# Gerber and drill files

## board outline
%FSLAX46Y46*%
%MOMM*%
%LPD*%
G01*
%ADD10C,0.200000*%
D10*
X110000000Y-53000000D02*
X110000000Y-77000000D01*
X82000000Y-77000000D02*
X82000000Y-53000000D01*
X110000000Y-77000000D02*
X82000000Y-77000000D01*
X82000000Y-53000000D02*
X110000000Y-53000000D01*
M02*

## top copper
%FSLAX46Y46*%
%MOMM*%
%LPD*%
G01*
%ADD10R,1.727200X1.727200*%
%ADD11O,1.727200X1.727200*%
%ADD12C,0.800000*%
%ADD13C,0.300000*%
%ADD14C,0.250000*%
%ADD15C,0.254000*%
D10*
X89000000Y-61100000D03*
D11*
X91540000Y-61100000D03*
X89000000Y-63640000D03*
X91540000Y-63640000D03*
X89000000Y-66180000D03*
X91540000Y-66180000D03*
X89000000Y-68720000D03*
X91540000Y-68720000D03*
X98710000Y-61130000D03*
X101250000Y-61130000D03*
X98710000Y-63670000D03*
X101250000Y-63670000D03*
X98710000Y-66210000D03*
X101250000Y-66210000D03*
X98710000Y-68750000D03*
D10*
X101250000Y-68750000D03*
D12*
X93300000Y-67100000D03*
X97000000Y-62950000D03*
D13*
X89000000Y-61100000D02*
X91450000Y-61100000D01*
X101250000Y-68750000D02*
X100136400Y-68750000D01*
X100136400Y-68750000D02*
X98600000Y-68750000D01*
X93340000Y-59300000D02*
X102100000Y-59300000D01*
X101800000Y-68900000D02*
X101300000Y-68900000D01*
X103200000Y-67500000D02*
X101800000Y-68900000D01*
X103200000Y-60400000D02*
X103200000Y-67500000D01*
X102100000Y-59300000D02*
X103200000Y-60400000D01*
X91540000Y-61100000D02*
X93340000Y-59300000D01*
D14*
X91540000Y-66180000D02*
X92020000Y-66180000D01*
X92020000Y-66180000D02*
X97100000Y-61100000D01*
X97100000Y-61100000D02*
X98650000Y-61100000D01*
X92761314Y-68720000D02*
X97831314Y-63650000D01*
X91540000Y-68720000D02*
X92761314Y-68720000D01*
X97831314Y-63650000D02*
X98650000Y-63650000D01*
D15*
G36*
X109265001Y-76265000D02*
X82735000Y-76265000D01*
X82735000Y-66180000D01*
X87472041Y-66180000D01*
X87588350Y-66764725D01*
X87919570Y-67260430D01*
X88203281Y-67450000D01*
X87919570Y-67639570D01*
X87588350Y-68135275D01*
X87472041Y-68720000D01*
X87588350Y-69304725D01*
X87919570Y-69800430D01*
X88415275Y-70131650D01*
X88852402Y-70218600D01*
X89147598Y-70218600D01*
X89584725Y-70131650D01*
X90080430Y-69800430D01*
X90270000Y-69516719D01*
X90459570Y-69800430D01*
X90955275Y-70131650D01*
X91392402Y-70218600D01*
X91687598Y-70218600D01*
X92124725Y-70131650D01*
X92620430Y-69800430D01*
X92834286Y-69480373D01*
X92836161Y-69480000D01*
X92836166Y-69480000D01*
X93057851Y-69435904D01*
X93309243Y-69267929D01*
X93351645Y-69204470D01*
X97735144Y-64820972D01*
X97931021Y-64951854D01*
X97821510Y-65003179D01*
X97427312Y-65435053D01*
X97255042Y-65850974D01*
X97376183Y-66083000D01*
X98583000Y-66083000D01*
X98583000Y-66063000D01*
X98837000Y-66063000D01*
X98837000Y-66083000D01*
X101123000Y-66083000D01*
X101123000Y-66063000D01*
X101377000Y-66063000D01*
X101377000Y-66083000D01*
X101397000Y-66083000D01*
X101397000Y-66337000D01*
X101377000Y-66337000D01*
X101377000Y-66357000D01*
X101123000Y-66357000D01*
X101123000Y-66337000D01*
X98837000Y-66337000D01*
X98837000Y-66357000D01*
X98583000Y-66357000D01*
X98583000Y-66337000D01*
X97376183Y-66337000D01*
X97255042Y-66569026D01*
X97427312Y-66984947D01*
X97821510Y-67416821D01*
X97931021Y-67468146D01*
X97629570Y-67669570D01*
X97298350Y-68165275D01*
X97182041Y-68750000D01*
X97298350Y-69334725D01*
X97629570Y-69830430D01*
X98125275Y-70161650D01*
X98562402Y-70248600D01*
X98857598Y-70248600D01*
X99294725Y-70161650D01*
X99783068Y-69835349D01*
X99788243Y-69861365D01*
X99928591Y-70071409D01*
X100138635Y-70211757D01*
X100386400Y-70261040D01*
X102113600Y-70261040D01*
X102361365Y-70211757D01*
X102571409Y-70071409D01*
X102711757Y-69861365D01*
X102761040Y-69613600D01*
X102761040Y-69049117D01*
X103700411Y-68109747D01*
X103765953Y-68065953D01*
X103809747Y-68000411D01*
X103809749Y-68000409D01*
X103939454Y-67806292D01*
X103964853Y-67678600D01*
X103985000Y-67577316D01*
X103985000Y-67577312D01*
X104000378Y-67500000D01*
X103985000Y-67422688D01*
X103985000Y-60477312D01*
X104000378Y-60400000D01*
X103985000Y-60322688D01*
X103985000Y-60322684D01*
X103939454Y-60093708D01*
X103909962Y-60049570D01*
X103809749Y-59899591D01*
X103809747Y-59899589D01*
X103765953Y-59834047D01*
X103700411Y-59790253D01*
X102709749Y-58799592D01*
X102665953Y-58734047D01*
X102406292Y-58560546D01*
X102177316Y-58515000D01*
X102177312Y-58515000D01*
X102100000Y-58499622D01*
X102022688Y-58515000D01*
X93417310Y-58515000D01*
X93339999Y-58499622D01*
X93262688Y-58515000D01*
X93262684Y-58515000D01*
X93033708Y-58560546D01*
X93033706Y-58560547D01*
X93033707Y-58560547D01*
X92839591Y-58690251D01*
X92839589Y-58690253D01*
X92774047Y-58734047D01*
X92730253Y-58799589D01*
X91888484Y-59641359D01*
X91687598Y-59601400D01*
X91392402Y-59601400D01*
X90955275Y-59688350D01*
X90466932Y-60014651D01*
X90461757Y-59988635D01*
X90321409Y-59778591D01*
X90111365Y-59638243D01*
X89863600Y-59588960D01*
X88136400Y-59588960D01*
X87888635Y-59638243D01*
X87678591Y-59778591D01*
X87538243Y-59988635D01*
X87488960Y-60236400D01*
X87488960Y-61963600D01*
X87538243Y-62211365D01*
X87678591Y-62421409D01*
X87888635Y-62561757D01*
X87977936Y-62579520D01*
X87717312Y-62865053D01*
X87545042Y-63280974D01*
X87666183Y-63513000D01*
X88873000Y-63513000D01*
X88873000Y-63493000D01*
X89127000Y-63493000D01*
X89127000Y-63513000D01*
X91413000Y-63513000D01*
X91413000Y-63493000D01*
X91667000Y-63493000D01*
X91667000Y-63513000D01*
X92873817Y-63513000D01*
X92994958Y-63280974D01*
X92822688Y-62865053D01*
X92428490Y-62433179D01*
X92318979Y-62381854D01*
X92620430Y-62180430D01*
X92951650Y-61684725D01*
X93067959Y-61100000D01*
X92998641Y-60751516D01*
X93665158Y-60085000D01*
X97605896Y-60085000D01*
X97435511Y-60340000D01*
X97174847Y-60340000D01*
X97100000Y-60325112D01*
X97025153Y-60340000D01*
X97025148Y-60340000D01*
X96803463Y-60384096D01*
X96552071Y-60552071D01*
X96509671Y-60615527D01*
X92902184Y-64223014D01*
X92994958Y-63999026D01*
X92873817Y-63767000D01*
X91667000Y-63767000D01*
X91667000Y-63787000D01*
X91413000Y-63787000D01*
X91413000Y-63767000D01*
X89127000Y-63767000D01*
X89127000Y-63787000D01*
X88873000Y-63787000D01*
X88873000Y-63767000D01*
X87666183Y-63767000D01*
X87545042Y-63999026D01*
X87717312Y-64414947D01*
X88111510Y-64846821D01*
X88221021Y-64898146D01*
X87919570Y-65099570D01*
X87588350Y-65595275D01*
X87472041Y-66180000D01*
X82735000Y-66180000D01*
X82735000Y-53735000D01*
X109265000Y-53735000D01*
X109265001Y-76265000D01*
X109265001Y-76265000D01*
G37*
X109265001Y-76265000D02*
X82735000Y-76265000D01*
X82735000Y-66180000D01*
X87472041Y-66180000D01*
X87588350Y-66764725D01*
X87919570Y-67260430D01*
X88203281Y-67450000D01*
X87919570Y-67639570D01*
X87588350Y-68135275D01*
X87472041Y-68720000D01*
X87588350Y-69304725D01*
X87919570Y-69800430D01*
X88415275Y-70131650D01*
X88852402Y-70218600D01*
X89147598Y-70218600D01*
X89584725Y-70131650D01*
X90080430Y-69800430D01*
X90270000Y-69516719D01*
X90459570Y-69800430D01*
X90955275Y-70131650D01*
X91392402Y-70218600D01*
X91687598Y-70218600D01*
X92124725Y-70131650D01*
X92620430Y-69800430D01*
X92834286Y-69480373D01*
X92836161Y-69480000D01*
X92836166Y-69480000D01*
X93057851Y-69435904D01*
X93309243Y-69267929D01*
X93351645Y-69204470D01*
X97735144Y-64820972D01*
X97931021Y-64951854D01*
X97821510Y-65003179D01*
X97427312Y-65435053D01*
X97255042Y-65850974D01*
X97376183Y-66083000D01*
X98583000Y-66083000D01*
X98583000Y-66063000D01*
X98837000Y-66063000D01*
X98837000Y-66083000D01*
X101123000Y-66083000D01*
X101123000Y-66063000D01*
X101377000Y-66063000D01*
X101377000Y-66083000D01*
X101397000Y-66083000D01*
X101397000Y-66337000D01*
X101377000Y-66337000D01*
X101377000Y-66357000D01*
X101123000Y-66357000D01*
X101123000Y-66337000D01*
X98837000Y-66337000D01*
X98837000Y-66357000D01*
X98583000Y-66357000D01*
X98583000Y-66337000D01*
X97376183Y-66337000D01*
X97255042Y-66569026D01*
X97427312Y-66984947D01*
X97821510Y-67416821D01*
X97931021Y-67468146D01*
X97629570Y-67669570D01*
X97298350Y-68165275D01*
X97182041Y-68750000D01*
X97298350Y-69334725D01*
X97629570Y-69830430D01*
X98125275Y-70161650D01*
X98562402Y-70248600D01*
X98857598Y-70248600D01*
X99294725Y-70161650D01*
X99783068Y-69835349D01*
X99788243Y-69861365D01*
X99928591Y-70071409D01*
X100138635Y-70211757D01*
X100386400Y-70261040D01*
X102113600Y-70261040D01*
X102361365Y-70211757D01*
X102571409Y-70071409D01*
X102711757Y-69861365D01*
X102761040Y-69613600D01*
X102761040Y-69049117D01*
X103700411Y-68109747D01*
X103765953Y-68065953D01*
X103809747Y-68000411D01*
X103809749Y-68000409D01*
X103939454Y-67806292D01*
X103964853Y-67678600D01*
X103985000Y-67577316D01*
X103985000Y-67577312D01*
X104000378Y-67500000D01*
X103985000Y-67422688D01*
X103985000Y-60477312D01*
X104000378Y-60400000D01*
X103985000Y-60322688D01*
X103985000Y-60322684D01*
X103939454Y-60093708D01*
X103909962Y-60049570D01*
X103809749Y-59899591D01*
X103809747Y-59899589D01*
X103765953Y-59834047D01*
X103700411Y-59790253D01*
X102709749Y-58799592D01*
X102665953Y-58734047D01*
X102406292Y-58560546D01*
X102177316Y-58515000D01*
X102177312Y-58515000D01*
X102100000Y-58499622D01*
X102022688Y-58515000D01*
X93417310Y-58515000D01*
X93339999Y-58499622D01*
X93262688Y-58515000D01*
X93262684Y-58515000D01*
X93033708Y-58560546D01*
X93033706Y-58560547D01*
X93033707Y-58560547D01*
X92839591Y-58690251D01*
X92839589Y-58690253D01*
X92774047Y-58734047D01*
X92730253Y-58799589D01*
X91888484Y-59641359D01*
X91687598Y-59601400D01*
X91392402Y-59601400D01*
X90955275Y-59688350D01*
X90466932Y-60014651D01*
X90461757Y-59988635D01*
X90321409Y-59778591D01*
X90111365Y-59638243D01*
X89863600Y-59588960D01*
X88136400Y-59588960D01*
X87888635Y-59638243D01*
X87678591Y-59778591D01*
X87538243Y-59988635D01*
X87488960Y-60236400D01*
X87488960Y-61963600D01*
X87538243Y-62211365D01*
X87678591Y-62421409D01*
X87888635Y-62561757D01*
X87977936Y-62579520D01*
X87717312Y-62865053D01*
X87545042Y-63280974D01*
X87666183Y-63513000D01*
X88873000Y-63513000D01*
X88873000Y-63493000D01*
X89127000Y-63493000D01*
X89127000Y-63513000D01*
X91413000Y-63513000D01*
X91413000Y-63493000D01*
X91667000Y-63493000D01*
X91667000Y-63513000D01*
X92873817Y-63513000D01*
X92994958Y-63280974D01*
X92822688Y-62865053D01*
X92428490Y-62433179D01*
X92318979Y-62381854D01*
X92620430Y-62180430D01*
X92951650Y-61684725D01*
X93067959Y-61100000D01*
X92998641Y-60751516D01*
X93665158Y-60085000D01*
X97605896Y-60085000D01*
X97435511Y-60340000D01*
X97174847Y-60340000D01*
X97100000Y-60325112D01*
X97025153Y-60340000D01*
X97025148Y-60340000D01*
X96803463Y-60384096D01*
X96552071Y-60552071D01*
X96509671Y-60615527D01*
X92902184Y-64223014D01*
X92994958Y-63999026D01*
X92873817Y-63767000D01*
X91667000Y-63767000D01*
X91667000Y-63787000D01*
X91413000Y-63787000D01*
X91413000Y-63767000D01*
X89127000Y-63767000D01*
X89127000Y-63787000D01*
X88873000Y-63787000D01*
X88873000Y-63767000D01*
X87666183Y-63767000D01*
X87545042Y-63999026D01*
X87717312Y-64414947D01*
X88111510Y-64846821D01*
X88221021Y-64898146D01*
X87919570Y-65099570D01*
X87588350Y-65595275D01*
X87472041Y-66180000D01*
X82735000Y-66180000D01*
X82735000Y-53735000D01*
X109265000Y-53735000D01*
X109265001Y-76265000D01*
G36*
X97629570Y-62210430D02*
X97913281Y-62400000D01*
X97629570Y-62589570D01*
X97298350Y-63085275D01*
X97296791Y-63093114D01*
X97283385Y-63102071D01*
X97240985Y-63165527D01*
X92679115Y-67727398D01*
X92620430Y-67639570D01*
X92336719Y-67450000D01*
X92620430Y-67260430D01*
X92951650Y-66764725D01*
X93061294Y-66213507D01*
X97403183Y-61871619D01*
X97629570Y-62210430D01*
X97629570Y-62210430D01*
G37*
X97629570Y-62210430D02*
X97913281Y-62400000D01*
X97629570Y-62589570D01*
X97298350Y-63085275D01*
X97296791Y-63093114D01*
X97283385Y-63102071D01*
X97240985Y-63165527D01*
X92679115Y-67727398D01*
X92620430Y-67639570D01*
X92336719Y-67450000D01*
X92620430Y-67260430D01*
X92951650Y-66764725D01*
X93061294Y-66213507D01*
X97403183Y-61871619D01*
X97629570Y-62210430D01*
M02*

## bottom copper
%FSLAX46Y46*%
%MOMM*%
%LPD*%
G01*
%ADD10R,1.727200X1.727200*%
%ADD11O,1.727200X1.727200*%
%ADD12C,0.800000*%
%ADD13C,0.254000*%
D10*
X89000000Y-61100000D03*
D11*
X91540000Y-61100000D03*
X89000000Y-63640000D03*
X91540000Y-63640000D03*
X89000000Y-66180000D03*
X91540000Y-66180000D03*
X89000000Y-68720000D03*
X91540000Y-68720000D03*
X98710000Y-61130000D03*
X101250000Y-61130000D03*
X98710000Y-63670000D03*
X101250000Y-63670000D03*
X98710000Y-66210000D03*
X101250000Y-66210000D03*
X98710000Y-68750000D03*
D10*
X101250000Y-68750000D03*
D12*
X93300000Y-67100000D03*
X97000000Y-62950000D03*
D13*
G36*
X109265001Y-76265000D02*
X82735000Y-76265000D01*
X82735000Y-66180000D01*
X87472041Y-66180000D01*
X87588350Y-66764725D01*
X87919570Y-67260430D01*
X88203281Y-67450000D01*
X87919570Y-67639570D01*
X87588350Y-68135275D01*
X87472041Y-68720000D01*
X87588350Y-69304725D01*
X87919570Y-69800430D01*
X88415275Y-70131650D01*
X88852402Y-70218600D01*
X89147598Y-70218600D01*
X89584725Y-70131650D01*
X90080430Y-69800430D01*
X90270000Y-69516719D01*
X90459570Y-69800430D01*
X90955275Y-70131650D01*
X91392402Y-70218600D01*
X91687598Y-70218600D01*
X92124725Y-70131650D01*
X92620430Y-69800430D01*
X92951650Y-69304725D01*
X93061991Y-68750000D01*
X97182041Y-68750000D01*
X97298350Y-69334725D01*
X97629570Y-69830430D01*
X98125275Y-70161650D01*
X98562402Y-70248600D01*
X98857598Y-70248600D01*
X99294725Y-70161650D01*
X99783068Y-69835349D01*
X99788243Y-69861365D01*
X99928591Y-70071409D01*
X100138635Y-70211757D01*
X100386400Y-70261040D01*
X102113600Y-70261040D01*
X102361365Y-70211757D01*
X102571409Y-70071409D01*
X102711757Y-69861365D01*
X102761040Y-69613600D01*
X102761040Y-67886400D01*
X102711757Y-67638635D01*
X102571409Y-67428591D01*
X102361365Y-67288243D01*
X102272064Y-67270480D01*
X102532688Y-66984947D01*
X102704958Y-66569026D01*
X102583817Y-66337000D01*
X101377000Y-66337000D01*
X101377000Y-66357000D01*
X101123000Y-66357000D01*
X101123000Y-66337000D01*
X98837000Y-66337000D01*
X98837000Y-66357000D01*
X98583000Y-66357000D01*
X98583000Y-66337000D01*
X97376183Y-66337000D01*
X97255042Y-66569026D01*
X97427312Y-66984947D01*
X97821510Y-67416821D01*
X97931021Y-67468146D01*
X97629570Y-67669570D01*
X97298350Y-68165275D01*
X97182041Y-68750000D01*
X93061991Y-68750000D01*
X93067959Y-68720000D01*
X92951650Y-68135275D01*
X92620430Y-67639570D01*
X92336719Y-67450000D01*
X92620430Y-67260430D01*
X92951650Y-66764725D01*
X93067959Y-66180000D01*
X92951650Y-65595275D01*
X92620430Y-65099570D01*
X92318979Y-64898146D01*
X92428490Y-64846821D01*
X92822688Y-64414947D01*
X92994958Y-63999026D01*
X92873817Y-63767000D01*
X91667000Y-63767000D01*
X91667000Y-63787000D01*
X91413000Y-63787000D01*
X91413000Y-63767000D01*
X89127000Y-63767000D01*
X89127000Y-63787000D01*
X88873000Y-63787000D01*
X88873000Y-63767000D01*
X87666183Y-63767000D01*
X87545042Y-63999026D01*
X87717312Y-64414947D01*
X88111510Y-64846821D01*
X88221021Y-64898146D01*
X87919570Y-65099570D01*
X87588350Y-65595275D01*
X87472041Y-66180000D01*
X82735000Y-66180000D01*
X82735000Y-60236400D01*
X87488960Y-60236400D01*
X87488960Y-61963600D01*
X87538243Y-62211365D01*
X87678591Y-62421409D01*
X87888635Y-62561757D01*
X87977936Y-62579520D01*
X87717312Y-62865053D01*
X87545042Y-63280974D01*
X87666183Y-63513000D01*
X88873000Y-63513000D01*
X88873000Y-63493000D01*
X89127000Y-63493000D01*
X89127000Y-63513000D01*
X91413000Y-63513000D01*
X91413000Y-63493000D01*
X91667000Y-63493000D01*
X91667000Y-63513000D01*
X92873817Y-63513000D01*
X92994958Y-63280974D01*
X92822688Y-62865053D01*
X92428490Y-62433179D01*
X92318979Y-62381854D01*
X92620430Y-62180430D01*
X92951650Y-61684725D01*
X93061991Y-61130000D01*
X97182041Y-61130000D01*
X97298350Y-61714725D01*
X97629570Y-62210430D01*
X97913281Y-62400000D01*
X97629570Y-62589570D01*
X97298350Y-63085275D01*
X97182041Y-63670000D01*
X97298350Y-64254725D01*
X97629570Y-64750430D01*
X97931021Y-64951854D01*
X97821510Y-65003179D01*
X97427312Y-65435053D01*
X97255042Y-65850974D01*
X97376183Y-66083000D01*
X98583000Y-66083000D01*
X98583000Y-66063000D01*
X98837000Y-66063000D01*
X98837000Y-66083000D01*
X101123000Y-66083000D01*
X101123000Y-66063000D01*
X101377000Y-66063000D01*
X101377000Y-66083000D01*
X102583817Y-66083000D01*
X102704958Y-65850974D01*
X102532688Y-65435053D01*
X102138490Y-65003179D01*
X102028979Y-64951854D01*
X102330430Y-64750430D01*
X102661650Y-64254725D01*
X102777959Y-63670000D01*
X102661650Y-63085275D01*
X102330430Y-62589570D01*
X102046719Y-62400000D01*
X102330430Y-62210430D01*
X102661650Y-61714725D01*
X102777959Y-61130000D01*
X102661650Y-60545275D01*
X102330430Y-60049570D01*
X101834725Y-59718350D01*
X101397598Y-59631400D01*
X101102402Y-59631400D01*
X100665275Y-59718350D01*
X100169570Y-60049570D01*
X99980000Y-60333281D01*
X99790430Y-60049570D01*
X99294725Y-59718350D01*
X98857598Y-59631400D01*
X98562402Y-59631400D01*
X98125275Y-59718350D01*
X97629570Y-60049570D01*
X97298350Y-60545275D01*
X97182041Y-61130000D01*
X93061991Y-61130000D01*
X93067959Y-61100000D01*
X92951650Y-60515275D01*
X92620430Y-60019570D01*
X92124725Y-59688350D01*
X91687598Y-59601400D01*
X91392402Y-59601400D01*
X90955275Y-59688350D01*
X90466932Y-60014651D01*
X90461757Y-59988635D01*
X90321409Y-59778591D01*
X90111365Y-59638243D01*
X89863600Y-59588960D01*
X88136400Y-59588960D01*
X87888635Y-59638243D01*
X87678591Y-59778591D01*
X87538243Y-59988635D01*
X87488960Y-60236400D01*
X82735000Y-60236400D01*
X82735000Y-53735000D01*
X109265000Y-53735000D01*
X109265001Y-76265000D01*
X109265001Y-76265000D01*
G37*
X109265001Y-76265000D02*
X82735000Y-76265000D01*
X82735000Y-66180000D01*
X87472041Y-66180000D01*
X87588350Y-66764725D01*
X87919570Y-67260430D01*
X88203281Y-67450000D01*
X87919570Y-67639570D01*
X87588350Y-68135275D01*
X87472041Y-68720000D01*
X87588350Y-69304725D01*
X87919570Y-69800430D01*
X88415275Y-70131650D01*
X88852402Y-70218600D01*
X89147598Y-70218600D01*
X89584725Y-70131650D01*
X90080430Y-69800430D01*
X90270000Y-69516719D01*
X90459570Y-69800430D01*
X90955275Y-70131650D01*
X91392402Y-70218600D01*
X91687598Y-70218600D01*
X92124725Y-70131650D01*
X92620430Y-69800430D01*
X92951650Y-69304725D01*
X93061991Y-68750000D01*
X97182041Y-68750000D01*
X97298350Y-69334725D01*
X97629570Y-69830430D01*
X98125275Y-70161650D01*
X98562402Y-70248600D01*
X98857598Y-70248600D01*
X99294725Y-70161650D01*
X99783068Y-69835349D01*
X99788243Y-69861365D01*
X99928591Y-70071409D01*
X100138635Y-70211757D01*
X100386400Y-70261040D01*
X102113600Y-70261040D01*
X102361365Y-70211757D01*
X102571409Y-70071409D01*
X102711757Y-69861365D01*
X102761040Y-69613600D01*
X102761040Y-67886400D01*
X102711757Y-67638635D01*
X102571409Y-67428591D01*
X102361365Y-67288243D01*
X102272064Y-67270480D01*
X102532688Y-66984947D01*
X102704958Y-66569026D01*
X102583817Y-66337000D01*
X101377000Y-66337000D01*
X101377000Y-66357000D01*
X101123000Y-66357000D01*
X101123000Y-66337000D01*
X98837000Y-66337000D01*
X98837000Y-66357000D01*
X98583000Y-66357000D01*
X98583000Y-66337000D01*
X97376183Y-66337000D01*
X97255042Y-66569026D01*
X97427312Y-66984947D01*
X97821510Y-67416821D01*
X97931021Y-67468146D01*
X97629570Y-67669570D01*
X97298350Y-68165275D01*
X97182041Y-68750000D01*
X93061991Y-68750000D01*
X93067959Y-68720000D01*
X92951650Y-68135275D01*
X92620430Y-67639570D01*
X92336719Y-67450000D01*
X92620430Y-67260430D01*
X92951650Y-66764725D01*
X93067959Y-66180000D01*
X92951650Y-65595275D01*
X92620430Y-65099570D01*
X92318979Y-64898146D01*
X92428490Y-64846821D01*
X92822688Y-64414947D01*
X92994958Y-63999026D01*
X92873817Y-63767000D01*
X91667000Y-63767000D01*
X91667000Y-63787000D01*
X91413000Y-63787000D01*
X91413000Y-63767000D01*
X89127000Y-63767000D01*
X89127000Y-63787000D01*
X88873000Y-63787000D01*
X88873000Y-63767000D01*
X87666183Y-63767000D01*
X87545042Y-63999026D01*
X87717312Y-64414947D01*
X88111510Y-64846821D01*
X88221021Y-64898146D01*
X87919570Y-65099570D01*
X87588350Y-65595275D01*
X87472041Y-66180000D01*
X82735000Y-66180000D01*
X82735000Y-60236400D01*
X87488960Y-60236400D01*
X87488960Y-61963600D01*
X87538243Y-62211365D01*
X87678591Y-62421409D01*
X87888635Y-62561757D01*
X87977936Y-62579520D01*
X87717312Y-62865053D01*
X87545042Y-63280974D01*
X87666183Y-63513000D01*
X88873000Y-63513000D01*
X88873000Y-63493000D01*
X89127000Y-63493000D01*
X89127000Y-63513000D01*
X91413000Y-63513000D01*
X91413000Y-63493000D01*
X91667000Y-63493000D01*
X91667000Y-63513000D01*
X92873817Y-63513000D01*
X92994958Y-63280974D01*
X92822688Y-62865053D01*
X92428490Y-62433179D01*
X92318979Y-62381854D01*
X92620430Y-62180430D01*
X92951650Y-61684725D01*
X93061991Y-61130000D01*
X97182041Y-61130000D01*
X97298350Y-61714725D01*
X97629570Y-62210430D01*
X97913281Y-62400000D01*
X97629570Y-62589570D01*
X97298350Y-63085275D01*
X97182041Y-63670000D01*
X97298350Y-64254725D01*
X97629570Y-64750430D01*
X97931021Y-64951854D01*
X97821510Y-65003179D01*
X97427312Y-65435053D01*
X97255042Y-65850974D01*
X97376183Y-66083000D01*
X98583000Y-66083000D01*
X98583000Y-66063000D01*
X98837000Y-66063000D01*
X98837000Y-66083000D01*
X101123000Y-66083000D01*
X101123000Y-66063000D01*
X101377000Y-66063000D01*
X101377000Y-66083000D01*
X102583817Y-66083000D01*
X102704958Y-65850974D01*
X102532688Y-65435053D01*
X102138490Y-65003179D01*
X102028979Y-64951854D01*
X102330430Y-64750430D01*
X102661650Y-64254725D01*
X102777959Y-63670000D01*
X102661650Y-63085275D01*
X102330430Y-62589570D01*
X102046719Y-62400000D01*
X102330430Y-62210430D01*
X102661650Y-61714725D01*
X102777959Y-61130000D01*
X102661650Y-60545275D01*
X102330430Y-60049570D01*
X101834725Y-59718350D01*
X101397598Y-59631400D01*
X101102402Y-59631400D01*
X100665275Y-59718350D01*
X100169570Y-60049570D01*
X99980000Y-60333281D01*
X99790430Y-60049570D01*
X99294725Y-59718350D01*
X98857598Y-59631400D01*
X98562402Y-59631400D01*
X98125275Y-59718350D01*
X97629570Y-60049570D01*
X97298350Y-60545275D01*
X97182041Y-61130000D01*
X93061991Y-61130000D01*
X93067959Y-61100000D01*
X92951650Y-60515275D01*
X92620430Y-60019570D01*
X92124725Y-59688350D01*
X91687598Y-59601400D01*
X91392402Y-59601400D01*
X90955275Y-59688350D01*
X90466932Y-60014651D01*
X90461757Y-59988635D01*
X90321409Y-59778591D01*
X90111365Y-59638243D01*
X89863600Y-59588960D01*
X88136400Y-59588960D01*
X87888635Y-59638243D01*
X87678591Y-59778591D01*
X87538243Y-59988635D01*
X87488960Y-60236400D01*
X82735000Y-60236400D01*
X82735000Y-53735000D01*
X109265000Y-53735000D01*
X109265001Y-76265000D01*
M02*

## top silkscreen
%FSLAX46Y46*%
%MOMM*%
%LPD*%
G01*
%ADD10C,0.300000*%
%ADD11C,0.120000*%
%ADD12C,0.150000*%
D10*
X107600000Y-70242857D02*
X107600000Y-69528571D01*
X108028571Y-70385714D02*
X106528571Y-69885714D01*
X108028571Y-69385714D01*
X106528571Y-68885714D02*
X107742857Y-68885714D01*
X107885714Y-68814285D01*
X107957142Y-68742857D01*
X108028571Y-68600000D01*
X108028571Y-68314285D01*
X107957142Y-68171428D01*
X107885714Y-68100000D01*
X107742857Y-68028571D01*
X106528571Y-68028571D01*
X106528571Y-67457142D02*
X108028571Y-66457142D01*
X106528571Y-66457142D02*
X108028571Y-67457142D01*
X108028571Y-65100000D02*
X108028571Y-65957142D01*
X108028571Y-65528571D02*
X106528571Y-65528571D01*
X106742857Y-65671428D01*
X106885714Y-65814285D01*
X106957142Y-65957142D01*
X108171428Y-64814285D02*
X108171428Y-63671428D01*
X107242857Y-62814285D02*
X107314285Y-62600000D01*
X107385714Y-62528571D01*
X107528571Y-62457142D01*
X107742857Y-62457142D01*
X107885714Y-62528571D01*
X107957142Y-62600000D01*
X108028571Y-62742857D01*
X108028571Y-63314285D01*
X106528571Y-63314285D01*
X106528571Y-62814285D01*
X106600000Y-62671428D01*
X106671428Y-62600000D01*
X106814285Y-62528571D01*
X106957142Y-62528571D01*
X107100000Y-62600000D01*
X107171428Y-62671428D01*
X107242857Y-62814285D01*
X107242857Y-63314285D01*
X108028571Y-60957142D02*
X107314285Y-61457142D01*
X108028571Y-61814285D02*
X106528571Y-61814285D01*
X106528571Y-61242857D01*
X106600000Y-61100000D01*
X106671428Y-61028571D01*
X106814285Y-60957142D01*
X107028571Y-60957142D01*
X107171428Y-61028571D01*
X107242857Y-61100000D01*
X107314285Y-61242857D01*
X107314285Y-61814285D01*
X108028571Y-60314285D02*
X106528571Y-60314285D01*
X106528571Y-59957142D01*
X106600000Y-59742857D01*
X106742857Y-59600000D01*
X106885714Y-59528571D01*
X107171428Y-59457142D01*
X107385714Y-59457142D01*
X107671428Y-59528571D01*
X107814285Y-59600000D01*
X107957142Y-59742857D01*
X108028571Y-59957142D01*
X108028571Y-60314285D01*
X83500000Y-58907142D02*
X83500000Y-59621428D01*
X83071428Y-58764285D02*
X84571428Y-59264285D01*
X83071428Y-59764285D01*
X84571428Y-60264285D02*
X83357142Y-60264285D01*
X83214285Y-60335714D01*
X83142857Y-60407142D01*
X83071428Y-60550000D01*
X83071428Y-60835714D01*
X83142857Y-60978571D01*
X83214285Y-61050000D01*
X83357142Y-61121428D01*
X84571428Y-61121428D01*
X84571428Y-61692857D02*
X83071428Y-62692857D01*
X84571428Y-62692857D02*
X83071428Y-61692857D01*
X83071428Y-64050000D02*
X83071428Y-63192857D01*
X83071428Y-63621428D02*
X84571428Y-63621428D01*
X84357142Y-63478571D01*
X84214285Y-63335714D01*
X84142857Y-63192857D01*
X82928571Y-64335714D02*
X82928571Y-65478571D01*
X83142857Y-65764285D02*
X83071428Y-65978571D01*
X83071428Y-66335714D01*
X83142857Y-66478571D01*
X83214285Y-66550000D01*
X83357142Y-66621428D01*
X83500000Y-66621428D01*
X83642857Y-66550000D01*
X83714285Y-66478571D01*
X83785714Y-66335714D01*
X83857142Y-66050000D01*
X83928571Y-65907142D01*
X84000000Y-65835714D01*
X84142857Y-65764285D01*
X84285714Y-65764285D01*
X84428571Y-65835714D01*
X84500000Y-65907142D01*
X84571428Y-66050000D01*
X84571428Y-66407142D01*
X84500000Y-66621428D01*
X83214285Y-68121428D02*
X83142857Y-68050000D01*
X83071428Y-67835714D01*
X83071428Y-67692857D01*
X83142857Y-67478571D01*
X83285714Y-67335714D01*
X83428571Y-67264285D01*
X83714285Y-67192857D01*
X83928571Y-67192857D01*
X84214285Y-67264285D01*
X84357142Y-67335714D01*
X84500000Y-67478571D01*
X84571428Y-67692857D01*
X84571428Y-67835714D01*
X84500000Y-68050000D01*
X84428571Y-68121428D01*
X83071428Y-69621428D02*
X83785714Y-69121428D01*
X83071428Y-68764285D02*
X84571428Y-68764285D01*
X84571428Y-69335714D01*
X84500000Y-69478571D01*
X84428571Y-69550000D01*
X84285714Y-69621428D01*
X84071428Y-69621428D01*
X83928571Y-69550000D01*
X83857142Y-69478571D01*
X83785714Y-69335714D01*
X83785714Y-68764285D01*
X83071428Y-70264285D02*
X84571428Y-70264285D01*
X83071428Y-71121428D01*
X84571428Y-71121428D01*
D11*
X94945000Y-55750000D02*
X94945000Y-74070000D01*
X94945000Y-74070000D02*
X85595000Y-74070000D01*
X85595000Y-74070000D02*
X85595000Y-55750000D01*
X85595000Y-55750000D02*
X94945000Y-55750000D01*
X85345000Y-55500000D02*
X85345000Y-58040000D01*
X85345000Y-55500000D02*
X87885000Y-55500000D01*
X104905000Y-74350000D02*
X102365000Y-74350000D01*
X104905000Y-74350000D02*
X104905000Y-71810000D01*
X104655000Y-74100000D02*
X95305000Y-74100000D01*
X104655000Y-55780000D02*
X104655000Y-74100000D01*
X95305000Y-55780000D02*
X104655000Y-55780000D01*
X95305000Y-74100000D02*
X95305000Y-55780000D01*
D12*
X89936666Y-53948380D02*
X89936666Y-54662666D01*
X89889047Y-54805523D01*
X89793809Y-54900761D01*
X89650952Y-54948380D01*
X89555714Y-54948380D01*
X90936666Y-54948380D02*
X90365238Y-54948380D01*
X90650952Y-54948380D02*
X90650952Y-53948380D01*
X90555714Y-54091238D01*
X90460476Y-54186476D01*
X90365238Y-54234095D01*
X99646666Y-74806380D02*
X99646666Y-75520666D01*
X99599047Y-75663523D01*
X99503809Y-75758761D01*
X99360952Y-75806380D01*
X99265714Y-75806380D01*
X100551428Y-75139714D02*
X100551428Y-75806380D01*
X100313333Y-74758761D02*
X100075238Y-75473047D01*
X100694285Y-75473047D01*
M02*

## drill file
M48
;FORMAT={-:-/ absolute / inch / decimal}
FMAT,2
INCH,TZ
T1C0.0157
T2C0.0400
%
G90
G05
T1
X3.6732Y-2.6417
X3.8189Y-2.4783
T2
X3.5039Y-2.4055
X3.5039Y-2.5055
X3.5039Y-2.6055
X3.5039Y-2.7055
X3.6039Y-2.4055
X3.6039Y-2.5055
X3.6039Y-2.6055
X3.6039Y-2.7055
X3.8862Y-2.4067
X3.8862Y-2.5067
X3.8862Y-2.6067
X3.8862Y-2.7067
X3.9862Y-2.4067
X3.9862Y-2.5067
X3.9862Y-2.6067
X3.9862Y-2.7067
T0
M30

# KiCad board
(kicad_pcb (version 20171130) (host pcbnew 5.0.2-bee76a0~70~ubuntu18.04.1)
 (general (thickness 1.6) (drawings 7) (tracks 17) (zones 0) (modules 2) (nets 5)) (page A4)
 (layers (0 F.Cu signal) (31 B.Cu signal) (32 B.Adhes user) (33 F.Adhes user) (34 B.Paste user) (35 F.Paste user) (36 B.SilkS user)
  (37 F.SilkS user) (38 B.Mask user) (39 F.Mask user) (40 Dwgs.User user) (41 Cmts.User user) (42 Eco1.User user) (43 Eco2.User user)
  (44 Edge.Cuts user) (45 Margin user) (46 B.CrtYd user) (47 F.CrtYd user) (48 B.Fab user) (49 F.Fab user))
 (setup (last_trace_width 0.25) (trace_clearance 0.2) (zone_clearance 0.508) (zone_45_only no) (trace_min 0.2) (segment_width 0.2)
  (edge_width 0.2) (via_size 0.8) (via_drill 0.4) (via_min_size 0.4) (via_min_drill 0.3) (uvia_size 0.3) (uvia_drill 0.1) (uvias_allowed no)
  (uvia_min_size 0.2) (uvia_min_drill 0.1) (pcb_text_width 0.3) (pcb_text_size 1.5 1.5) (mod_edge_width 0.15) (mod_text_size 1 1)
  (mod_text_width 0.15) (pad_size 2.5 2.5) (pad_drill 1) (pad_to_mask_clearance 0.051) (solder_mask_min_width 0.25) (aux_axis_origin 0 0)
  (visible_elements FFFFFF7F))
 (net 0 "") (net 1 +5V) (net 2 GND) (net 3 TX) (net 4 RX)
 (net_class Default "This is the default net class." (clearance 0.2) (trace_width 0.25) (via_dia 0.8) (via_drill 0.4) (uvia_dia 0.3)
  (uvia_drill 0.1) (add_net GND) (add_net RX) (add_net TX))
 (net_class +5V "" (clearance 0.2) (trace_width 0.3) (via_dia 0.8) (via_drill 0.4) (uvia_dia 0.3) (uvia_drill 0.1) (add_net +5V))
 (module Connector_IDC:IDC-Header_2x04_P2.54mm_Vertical (layer F.Cu) (at 89 61.1)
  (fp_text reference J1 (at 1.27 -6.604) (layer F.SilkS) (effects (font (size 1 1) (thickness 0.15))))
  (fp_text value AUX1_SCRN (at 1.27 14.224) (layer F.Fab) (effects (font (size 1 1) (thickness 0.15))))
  (fp_line (start 5.945 -5.35) (end 5.945 12.97) (layer F.SilkS) (width 0.12))
  (fp_line (start 5.945 12.97) (end -3.405 12.97) (layer F.SilkS) (width 0.12))
  (fp_line (start -3.405 12.97) (end -3.405 -5.35) (layer F.SilkS) (width 0.12))
  (fp_line (start -3.405 -5.35) (end 5.945 -5.35) (layer F.SilkS) (width 0.12))
  (fp_line (start -3.655 -5.6) (end -3.655 -3.06) (layer F.SilkS) (width 0.12))
  (fp_line (start -3.655 -5.6) (end -1.115 -5.6) (layer F.SilkS) (width 0.12))
  (pad 1 thru_hole rect (at 0 0) (size 1.7272 1.7272) (drill 1.016) (layers *.Cu *.Mask) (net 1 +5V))
  (pad 2 thru_hole oval (at 2.54 0) (size 1.7272 1.7272) (drill 1.016) (layers *.Cu *.Mask) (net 1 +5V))
  (pad 3 thru_hole oval (at 0 2.54) (size 1.7272 1.7272) (drill 1.016) (layers *.Cu *.Mask) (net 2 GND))
  (pad 4 thru_hole oval (at 2.54 2.54) (size 1.7272 1.7272) (drill 1.016) (layers *.Cu *.Mask) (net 2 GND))
  (pad 5 thru_hole oval (at 0 5.08) (size 1.7272 1.7272) (drill 1.016) (layers *.Cu *.Mask))
  (pad 6 thru_hole oval (at 2.54 5.08) (size 1.7272 1.7272) (drill 1.016) (layers *.Cu *.Mask) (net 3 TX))
  (pad 7 thru_hole oval (at 0 7.62) (size 1.7272 1.7272) (drill 1.016) (layers *.Cu *.Mask))
  (pad 8 thru_hole oval (at 2.54 7.62) (size 1.7272 1.7272) (drill 1.016) (layers *.Cu *.Mask) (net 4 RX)))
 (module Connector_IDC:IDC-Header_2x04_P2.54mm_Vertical (layer F.Cu) (at 101.25 68.75 180)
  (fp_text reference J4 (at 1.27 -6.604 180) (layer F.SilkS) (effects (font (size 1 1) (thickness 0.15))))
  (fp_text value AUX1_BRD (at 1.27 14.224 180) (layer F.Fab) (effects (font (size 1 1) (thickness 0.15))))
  (fp_line (start -3.655 -5.6) (end -1.115 -5.6) (layer F.SilkS) (width 0.12))
  (fp_line (start -3.655 -5.6) (end -3.655 -3.06) (layer F.SilkS) (width 0.12))
  (fp_line (start -3.405 -5.35) (end 5.945 -5.35) (layer F.SilkS) (width 0.12))
  (fp_line (start -3.405 12.97) (end -3.405 -5.35) (layer F.SilkS) (width 0.12))
  (fp_line (start 5.945 12.97) (end -3.405 12.97) (layer F.SilkS) (width 0.12))
  (fp_line (start 5.945 -5.35) (end 5.945 12.97) (layer F.SilkS) (width 0.12))
  (pad 8 thru_hole oval (at 2.54 7.62 180) (size 1.7272 1.7272) (drill 1.016) (layers *.Cu *.Mask) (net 3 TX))
  (pad 7 thru_hole oval (at 0 7.62 180) (size 1.7272 1.7272) (drill 1.016) (layers *.Cu *.Mask))
  (pad 6 thru_hole oval (at 2.54 5.08 180) (size 1.7272 1.7272) (drill 1.016) (layers *.Cu *.Mask) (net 4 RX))
  (pad 5 thru_hole oval (at 0 5.08 180) (size 1.7272 1.7272) (drill 1.016) (layers *.Cu *.Mask))
  (pad 4 thru_hole oval (at 2.54 2.54 180) (size 1.7272 1.7272) (drill 1.016) (layers *.Cu *.Mask) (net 2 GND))
  (pad 3 thru_hole oval (at 0 2.54 180) (size 1.7272 1.7272) (drill 1.016) (layers *.Cu *.Mask) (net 2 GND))
  (pad 2 thru_hole oval (at 2.54 0 180) (size 1.7272 1.7272) (drill 1.016) (layers *.Cu *.Mask) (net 1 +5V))
  (pad 1 thru_hole rect (at 0 0 180) (size 1.7272 1.7272) (drill 1.016) (layers *.Cu *.Mask) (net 1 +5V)))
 (gr_line (start 110 53) (end 110 77) (layer Edge.Cuts) (width 0.2))
 (gr_line (start 82 77) (end 82 53) (layer Edge.Cuts) (width 0.2))
 (gr_line (start 110 77) (end 82 77) (layer Edge.Cuts) (width 0.2))
 (gr_line (start 82 53) (end 110 53) (layer Edge.Cuts) (width 0.2))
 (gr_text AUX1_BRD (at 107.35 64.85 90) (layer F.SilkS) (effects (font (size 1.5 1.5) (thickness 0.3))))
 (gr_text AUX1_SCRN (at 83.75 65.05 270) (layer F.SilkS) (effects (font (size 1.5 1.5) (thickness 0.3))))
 (segment (start 89 61.1) (end 91.45 61.1) (width 0.3) (layer F.Cu) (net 1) (status 30))
 (segment (start 101.25 68.75) (end 100.1364 68.75) (width 0.3) (layer F.Cu) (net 1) (status 10))
 (segment (start 100.1364 68.75) (end 98.6 68.75) (width 0.3) (layer F.Cu) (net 1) (status 20))
 (segment (start 93.34 59.3) (end 102.1 59.3) (width 0.3) (layer F.Cu) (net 1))
 (segment (start 101.8 68.9) (end 101.3 68.9) (width 0.3) (layer F.Cu) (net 1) (status 30))
 (segment (start 103.2 67.5) (end 101.8 68.9) (width 0.3) (layer F.Cu) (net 1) (status 20))
 (segment (start 103.2 60.4) (end 103.2 67.5) (width 0.3) (layer F.Cu) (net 1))
 (segment (start 102.1 59.3) (end 103.2 60.4) (width 0.3) (layer F.Cu) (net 1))
 (segment (start 91.54 61.1) (end 93.34 59.3) (width 0.3) (layer F.Cu) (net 1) (status 10))
 (via (at 93.3 67.1) (size 0.8) (drill 0.4) (layers F.Cu B.Cu) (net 2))
 (via (at 97 62.95) (size 0.8) (drill 0.4) (layers F.Cu B.Cu) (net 2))
 (segment (start 91.54 66.18) (end 92.02 66.18) (width 0.25) (layer F.Cu) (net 3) (status 30))
 (segment (start 92.02 66.18) (end 97.1 61.1) (width 0.25) (layer F.Cu) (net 3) (status 10))
 (segment (start 97.1 61.1) (end 98.65 61.1) (width 0.25) (layer F.Cu) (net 3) (status 20))
 (segment (start 92.761314 68.72) (end 97.831314 63.65) (width 0.25) (layer F.Cu) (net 4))
 (segment (start 91.54 68.72) (end 92.761314 68.72) (width 0.25) (layer F.Cu) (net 4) (status 10))
 (segment (start 97.831314 63.65) (end 98.65 63.65) (width 0.25) (layer F.Cu) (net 4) (status 20))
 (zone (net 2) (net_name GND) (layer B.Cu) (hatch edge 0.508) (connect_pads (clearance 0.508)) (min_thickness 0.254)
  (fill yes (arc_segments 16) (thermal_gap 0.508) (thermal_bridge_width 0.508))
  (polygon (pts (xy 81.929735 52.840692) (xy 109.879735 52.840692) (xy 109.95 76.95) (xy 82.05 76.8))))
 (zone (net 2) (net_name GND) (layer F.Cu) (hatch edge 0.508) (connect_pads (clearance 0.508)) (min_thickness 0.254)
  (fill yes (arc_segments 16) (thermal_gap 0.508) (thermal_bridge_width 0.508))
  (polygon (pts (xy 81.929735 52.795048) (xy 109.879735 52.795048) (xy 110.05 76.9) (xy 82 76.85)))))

